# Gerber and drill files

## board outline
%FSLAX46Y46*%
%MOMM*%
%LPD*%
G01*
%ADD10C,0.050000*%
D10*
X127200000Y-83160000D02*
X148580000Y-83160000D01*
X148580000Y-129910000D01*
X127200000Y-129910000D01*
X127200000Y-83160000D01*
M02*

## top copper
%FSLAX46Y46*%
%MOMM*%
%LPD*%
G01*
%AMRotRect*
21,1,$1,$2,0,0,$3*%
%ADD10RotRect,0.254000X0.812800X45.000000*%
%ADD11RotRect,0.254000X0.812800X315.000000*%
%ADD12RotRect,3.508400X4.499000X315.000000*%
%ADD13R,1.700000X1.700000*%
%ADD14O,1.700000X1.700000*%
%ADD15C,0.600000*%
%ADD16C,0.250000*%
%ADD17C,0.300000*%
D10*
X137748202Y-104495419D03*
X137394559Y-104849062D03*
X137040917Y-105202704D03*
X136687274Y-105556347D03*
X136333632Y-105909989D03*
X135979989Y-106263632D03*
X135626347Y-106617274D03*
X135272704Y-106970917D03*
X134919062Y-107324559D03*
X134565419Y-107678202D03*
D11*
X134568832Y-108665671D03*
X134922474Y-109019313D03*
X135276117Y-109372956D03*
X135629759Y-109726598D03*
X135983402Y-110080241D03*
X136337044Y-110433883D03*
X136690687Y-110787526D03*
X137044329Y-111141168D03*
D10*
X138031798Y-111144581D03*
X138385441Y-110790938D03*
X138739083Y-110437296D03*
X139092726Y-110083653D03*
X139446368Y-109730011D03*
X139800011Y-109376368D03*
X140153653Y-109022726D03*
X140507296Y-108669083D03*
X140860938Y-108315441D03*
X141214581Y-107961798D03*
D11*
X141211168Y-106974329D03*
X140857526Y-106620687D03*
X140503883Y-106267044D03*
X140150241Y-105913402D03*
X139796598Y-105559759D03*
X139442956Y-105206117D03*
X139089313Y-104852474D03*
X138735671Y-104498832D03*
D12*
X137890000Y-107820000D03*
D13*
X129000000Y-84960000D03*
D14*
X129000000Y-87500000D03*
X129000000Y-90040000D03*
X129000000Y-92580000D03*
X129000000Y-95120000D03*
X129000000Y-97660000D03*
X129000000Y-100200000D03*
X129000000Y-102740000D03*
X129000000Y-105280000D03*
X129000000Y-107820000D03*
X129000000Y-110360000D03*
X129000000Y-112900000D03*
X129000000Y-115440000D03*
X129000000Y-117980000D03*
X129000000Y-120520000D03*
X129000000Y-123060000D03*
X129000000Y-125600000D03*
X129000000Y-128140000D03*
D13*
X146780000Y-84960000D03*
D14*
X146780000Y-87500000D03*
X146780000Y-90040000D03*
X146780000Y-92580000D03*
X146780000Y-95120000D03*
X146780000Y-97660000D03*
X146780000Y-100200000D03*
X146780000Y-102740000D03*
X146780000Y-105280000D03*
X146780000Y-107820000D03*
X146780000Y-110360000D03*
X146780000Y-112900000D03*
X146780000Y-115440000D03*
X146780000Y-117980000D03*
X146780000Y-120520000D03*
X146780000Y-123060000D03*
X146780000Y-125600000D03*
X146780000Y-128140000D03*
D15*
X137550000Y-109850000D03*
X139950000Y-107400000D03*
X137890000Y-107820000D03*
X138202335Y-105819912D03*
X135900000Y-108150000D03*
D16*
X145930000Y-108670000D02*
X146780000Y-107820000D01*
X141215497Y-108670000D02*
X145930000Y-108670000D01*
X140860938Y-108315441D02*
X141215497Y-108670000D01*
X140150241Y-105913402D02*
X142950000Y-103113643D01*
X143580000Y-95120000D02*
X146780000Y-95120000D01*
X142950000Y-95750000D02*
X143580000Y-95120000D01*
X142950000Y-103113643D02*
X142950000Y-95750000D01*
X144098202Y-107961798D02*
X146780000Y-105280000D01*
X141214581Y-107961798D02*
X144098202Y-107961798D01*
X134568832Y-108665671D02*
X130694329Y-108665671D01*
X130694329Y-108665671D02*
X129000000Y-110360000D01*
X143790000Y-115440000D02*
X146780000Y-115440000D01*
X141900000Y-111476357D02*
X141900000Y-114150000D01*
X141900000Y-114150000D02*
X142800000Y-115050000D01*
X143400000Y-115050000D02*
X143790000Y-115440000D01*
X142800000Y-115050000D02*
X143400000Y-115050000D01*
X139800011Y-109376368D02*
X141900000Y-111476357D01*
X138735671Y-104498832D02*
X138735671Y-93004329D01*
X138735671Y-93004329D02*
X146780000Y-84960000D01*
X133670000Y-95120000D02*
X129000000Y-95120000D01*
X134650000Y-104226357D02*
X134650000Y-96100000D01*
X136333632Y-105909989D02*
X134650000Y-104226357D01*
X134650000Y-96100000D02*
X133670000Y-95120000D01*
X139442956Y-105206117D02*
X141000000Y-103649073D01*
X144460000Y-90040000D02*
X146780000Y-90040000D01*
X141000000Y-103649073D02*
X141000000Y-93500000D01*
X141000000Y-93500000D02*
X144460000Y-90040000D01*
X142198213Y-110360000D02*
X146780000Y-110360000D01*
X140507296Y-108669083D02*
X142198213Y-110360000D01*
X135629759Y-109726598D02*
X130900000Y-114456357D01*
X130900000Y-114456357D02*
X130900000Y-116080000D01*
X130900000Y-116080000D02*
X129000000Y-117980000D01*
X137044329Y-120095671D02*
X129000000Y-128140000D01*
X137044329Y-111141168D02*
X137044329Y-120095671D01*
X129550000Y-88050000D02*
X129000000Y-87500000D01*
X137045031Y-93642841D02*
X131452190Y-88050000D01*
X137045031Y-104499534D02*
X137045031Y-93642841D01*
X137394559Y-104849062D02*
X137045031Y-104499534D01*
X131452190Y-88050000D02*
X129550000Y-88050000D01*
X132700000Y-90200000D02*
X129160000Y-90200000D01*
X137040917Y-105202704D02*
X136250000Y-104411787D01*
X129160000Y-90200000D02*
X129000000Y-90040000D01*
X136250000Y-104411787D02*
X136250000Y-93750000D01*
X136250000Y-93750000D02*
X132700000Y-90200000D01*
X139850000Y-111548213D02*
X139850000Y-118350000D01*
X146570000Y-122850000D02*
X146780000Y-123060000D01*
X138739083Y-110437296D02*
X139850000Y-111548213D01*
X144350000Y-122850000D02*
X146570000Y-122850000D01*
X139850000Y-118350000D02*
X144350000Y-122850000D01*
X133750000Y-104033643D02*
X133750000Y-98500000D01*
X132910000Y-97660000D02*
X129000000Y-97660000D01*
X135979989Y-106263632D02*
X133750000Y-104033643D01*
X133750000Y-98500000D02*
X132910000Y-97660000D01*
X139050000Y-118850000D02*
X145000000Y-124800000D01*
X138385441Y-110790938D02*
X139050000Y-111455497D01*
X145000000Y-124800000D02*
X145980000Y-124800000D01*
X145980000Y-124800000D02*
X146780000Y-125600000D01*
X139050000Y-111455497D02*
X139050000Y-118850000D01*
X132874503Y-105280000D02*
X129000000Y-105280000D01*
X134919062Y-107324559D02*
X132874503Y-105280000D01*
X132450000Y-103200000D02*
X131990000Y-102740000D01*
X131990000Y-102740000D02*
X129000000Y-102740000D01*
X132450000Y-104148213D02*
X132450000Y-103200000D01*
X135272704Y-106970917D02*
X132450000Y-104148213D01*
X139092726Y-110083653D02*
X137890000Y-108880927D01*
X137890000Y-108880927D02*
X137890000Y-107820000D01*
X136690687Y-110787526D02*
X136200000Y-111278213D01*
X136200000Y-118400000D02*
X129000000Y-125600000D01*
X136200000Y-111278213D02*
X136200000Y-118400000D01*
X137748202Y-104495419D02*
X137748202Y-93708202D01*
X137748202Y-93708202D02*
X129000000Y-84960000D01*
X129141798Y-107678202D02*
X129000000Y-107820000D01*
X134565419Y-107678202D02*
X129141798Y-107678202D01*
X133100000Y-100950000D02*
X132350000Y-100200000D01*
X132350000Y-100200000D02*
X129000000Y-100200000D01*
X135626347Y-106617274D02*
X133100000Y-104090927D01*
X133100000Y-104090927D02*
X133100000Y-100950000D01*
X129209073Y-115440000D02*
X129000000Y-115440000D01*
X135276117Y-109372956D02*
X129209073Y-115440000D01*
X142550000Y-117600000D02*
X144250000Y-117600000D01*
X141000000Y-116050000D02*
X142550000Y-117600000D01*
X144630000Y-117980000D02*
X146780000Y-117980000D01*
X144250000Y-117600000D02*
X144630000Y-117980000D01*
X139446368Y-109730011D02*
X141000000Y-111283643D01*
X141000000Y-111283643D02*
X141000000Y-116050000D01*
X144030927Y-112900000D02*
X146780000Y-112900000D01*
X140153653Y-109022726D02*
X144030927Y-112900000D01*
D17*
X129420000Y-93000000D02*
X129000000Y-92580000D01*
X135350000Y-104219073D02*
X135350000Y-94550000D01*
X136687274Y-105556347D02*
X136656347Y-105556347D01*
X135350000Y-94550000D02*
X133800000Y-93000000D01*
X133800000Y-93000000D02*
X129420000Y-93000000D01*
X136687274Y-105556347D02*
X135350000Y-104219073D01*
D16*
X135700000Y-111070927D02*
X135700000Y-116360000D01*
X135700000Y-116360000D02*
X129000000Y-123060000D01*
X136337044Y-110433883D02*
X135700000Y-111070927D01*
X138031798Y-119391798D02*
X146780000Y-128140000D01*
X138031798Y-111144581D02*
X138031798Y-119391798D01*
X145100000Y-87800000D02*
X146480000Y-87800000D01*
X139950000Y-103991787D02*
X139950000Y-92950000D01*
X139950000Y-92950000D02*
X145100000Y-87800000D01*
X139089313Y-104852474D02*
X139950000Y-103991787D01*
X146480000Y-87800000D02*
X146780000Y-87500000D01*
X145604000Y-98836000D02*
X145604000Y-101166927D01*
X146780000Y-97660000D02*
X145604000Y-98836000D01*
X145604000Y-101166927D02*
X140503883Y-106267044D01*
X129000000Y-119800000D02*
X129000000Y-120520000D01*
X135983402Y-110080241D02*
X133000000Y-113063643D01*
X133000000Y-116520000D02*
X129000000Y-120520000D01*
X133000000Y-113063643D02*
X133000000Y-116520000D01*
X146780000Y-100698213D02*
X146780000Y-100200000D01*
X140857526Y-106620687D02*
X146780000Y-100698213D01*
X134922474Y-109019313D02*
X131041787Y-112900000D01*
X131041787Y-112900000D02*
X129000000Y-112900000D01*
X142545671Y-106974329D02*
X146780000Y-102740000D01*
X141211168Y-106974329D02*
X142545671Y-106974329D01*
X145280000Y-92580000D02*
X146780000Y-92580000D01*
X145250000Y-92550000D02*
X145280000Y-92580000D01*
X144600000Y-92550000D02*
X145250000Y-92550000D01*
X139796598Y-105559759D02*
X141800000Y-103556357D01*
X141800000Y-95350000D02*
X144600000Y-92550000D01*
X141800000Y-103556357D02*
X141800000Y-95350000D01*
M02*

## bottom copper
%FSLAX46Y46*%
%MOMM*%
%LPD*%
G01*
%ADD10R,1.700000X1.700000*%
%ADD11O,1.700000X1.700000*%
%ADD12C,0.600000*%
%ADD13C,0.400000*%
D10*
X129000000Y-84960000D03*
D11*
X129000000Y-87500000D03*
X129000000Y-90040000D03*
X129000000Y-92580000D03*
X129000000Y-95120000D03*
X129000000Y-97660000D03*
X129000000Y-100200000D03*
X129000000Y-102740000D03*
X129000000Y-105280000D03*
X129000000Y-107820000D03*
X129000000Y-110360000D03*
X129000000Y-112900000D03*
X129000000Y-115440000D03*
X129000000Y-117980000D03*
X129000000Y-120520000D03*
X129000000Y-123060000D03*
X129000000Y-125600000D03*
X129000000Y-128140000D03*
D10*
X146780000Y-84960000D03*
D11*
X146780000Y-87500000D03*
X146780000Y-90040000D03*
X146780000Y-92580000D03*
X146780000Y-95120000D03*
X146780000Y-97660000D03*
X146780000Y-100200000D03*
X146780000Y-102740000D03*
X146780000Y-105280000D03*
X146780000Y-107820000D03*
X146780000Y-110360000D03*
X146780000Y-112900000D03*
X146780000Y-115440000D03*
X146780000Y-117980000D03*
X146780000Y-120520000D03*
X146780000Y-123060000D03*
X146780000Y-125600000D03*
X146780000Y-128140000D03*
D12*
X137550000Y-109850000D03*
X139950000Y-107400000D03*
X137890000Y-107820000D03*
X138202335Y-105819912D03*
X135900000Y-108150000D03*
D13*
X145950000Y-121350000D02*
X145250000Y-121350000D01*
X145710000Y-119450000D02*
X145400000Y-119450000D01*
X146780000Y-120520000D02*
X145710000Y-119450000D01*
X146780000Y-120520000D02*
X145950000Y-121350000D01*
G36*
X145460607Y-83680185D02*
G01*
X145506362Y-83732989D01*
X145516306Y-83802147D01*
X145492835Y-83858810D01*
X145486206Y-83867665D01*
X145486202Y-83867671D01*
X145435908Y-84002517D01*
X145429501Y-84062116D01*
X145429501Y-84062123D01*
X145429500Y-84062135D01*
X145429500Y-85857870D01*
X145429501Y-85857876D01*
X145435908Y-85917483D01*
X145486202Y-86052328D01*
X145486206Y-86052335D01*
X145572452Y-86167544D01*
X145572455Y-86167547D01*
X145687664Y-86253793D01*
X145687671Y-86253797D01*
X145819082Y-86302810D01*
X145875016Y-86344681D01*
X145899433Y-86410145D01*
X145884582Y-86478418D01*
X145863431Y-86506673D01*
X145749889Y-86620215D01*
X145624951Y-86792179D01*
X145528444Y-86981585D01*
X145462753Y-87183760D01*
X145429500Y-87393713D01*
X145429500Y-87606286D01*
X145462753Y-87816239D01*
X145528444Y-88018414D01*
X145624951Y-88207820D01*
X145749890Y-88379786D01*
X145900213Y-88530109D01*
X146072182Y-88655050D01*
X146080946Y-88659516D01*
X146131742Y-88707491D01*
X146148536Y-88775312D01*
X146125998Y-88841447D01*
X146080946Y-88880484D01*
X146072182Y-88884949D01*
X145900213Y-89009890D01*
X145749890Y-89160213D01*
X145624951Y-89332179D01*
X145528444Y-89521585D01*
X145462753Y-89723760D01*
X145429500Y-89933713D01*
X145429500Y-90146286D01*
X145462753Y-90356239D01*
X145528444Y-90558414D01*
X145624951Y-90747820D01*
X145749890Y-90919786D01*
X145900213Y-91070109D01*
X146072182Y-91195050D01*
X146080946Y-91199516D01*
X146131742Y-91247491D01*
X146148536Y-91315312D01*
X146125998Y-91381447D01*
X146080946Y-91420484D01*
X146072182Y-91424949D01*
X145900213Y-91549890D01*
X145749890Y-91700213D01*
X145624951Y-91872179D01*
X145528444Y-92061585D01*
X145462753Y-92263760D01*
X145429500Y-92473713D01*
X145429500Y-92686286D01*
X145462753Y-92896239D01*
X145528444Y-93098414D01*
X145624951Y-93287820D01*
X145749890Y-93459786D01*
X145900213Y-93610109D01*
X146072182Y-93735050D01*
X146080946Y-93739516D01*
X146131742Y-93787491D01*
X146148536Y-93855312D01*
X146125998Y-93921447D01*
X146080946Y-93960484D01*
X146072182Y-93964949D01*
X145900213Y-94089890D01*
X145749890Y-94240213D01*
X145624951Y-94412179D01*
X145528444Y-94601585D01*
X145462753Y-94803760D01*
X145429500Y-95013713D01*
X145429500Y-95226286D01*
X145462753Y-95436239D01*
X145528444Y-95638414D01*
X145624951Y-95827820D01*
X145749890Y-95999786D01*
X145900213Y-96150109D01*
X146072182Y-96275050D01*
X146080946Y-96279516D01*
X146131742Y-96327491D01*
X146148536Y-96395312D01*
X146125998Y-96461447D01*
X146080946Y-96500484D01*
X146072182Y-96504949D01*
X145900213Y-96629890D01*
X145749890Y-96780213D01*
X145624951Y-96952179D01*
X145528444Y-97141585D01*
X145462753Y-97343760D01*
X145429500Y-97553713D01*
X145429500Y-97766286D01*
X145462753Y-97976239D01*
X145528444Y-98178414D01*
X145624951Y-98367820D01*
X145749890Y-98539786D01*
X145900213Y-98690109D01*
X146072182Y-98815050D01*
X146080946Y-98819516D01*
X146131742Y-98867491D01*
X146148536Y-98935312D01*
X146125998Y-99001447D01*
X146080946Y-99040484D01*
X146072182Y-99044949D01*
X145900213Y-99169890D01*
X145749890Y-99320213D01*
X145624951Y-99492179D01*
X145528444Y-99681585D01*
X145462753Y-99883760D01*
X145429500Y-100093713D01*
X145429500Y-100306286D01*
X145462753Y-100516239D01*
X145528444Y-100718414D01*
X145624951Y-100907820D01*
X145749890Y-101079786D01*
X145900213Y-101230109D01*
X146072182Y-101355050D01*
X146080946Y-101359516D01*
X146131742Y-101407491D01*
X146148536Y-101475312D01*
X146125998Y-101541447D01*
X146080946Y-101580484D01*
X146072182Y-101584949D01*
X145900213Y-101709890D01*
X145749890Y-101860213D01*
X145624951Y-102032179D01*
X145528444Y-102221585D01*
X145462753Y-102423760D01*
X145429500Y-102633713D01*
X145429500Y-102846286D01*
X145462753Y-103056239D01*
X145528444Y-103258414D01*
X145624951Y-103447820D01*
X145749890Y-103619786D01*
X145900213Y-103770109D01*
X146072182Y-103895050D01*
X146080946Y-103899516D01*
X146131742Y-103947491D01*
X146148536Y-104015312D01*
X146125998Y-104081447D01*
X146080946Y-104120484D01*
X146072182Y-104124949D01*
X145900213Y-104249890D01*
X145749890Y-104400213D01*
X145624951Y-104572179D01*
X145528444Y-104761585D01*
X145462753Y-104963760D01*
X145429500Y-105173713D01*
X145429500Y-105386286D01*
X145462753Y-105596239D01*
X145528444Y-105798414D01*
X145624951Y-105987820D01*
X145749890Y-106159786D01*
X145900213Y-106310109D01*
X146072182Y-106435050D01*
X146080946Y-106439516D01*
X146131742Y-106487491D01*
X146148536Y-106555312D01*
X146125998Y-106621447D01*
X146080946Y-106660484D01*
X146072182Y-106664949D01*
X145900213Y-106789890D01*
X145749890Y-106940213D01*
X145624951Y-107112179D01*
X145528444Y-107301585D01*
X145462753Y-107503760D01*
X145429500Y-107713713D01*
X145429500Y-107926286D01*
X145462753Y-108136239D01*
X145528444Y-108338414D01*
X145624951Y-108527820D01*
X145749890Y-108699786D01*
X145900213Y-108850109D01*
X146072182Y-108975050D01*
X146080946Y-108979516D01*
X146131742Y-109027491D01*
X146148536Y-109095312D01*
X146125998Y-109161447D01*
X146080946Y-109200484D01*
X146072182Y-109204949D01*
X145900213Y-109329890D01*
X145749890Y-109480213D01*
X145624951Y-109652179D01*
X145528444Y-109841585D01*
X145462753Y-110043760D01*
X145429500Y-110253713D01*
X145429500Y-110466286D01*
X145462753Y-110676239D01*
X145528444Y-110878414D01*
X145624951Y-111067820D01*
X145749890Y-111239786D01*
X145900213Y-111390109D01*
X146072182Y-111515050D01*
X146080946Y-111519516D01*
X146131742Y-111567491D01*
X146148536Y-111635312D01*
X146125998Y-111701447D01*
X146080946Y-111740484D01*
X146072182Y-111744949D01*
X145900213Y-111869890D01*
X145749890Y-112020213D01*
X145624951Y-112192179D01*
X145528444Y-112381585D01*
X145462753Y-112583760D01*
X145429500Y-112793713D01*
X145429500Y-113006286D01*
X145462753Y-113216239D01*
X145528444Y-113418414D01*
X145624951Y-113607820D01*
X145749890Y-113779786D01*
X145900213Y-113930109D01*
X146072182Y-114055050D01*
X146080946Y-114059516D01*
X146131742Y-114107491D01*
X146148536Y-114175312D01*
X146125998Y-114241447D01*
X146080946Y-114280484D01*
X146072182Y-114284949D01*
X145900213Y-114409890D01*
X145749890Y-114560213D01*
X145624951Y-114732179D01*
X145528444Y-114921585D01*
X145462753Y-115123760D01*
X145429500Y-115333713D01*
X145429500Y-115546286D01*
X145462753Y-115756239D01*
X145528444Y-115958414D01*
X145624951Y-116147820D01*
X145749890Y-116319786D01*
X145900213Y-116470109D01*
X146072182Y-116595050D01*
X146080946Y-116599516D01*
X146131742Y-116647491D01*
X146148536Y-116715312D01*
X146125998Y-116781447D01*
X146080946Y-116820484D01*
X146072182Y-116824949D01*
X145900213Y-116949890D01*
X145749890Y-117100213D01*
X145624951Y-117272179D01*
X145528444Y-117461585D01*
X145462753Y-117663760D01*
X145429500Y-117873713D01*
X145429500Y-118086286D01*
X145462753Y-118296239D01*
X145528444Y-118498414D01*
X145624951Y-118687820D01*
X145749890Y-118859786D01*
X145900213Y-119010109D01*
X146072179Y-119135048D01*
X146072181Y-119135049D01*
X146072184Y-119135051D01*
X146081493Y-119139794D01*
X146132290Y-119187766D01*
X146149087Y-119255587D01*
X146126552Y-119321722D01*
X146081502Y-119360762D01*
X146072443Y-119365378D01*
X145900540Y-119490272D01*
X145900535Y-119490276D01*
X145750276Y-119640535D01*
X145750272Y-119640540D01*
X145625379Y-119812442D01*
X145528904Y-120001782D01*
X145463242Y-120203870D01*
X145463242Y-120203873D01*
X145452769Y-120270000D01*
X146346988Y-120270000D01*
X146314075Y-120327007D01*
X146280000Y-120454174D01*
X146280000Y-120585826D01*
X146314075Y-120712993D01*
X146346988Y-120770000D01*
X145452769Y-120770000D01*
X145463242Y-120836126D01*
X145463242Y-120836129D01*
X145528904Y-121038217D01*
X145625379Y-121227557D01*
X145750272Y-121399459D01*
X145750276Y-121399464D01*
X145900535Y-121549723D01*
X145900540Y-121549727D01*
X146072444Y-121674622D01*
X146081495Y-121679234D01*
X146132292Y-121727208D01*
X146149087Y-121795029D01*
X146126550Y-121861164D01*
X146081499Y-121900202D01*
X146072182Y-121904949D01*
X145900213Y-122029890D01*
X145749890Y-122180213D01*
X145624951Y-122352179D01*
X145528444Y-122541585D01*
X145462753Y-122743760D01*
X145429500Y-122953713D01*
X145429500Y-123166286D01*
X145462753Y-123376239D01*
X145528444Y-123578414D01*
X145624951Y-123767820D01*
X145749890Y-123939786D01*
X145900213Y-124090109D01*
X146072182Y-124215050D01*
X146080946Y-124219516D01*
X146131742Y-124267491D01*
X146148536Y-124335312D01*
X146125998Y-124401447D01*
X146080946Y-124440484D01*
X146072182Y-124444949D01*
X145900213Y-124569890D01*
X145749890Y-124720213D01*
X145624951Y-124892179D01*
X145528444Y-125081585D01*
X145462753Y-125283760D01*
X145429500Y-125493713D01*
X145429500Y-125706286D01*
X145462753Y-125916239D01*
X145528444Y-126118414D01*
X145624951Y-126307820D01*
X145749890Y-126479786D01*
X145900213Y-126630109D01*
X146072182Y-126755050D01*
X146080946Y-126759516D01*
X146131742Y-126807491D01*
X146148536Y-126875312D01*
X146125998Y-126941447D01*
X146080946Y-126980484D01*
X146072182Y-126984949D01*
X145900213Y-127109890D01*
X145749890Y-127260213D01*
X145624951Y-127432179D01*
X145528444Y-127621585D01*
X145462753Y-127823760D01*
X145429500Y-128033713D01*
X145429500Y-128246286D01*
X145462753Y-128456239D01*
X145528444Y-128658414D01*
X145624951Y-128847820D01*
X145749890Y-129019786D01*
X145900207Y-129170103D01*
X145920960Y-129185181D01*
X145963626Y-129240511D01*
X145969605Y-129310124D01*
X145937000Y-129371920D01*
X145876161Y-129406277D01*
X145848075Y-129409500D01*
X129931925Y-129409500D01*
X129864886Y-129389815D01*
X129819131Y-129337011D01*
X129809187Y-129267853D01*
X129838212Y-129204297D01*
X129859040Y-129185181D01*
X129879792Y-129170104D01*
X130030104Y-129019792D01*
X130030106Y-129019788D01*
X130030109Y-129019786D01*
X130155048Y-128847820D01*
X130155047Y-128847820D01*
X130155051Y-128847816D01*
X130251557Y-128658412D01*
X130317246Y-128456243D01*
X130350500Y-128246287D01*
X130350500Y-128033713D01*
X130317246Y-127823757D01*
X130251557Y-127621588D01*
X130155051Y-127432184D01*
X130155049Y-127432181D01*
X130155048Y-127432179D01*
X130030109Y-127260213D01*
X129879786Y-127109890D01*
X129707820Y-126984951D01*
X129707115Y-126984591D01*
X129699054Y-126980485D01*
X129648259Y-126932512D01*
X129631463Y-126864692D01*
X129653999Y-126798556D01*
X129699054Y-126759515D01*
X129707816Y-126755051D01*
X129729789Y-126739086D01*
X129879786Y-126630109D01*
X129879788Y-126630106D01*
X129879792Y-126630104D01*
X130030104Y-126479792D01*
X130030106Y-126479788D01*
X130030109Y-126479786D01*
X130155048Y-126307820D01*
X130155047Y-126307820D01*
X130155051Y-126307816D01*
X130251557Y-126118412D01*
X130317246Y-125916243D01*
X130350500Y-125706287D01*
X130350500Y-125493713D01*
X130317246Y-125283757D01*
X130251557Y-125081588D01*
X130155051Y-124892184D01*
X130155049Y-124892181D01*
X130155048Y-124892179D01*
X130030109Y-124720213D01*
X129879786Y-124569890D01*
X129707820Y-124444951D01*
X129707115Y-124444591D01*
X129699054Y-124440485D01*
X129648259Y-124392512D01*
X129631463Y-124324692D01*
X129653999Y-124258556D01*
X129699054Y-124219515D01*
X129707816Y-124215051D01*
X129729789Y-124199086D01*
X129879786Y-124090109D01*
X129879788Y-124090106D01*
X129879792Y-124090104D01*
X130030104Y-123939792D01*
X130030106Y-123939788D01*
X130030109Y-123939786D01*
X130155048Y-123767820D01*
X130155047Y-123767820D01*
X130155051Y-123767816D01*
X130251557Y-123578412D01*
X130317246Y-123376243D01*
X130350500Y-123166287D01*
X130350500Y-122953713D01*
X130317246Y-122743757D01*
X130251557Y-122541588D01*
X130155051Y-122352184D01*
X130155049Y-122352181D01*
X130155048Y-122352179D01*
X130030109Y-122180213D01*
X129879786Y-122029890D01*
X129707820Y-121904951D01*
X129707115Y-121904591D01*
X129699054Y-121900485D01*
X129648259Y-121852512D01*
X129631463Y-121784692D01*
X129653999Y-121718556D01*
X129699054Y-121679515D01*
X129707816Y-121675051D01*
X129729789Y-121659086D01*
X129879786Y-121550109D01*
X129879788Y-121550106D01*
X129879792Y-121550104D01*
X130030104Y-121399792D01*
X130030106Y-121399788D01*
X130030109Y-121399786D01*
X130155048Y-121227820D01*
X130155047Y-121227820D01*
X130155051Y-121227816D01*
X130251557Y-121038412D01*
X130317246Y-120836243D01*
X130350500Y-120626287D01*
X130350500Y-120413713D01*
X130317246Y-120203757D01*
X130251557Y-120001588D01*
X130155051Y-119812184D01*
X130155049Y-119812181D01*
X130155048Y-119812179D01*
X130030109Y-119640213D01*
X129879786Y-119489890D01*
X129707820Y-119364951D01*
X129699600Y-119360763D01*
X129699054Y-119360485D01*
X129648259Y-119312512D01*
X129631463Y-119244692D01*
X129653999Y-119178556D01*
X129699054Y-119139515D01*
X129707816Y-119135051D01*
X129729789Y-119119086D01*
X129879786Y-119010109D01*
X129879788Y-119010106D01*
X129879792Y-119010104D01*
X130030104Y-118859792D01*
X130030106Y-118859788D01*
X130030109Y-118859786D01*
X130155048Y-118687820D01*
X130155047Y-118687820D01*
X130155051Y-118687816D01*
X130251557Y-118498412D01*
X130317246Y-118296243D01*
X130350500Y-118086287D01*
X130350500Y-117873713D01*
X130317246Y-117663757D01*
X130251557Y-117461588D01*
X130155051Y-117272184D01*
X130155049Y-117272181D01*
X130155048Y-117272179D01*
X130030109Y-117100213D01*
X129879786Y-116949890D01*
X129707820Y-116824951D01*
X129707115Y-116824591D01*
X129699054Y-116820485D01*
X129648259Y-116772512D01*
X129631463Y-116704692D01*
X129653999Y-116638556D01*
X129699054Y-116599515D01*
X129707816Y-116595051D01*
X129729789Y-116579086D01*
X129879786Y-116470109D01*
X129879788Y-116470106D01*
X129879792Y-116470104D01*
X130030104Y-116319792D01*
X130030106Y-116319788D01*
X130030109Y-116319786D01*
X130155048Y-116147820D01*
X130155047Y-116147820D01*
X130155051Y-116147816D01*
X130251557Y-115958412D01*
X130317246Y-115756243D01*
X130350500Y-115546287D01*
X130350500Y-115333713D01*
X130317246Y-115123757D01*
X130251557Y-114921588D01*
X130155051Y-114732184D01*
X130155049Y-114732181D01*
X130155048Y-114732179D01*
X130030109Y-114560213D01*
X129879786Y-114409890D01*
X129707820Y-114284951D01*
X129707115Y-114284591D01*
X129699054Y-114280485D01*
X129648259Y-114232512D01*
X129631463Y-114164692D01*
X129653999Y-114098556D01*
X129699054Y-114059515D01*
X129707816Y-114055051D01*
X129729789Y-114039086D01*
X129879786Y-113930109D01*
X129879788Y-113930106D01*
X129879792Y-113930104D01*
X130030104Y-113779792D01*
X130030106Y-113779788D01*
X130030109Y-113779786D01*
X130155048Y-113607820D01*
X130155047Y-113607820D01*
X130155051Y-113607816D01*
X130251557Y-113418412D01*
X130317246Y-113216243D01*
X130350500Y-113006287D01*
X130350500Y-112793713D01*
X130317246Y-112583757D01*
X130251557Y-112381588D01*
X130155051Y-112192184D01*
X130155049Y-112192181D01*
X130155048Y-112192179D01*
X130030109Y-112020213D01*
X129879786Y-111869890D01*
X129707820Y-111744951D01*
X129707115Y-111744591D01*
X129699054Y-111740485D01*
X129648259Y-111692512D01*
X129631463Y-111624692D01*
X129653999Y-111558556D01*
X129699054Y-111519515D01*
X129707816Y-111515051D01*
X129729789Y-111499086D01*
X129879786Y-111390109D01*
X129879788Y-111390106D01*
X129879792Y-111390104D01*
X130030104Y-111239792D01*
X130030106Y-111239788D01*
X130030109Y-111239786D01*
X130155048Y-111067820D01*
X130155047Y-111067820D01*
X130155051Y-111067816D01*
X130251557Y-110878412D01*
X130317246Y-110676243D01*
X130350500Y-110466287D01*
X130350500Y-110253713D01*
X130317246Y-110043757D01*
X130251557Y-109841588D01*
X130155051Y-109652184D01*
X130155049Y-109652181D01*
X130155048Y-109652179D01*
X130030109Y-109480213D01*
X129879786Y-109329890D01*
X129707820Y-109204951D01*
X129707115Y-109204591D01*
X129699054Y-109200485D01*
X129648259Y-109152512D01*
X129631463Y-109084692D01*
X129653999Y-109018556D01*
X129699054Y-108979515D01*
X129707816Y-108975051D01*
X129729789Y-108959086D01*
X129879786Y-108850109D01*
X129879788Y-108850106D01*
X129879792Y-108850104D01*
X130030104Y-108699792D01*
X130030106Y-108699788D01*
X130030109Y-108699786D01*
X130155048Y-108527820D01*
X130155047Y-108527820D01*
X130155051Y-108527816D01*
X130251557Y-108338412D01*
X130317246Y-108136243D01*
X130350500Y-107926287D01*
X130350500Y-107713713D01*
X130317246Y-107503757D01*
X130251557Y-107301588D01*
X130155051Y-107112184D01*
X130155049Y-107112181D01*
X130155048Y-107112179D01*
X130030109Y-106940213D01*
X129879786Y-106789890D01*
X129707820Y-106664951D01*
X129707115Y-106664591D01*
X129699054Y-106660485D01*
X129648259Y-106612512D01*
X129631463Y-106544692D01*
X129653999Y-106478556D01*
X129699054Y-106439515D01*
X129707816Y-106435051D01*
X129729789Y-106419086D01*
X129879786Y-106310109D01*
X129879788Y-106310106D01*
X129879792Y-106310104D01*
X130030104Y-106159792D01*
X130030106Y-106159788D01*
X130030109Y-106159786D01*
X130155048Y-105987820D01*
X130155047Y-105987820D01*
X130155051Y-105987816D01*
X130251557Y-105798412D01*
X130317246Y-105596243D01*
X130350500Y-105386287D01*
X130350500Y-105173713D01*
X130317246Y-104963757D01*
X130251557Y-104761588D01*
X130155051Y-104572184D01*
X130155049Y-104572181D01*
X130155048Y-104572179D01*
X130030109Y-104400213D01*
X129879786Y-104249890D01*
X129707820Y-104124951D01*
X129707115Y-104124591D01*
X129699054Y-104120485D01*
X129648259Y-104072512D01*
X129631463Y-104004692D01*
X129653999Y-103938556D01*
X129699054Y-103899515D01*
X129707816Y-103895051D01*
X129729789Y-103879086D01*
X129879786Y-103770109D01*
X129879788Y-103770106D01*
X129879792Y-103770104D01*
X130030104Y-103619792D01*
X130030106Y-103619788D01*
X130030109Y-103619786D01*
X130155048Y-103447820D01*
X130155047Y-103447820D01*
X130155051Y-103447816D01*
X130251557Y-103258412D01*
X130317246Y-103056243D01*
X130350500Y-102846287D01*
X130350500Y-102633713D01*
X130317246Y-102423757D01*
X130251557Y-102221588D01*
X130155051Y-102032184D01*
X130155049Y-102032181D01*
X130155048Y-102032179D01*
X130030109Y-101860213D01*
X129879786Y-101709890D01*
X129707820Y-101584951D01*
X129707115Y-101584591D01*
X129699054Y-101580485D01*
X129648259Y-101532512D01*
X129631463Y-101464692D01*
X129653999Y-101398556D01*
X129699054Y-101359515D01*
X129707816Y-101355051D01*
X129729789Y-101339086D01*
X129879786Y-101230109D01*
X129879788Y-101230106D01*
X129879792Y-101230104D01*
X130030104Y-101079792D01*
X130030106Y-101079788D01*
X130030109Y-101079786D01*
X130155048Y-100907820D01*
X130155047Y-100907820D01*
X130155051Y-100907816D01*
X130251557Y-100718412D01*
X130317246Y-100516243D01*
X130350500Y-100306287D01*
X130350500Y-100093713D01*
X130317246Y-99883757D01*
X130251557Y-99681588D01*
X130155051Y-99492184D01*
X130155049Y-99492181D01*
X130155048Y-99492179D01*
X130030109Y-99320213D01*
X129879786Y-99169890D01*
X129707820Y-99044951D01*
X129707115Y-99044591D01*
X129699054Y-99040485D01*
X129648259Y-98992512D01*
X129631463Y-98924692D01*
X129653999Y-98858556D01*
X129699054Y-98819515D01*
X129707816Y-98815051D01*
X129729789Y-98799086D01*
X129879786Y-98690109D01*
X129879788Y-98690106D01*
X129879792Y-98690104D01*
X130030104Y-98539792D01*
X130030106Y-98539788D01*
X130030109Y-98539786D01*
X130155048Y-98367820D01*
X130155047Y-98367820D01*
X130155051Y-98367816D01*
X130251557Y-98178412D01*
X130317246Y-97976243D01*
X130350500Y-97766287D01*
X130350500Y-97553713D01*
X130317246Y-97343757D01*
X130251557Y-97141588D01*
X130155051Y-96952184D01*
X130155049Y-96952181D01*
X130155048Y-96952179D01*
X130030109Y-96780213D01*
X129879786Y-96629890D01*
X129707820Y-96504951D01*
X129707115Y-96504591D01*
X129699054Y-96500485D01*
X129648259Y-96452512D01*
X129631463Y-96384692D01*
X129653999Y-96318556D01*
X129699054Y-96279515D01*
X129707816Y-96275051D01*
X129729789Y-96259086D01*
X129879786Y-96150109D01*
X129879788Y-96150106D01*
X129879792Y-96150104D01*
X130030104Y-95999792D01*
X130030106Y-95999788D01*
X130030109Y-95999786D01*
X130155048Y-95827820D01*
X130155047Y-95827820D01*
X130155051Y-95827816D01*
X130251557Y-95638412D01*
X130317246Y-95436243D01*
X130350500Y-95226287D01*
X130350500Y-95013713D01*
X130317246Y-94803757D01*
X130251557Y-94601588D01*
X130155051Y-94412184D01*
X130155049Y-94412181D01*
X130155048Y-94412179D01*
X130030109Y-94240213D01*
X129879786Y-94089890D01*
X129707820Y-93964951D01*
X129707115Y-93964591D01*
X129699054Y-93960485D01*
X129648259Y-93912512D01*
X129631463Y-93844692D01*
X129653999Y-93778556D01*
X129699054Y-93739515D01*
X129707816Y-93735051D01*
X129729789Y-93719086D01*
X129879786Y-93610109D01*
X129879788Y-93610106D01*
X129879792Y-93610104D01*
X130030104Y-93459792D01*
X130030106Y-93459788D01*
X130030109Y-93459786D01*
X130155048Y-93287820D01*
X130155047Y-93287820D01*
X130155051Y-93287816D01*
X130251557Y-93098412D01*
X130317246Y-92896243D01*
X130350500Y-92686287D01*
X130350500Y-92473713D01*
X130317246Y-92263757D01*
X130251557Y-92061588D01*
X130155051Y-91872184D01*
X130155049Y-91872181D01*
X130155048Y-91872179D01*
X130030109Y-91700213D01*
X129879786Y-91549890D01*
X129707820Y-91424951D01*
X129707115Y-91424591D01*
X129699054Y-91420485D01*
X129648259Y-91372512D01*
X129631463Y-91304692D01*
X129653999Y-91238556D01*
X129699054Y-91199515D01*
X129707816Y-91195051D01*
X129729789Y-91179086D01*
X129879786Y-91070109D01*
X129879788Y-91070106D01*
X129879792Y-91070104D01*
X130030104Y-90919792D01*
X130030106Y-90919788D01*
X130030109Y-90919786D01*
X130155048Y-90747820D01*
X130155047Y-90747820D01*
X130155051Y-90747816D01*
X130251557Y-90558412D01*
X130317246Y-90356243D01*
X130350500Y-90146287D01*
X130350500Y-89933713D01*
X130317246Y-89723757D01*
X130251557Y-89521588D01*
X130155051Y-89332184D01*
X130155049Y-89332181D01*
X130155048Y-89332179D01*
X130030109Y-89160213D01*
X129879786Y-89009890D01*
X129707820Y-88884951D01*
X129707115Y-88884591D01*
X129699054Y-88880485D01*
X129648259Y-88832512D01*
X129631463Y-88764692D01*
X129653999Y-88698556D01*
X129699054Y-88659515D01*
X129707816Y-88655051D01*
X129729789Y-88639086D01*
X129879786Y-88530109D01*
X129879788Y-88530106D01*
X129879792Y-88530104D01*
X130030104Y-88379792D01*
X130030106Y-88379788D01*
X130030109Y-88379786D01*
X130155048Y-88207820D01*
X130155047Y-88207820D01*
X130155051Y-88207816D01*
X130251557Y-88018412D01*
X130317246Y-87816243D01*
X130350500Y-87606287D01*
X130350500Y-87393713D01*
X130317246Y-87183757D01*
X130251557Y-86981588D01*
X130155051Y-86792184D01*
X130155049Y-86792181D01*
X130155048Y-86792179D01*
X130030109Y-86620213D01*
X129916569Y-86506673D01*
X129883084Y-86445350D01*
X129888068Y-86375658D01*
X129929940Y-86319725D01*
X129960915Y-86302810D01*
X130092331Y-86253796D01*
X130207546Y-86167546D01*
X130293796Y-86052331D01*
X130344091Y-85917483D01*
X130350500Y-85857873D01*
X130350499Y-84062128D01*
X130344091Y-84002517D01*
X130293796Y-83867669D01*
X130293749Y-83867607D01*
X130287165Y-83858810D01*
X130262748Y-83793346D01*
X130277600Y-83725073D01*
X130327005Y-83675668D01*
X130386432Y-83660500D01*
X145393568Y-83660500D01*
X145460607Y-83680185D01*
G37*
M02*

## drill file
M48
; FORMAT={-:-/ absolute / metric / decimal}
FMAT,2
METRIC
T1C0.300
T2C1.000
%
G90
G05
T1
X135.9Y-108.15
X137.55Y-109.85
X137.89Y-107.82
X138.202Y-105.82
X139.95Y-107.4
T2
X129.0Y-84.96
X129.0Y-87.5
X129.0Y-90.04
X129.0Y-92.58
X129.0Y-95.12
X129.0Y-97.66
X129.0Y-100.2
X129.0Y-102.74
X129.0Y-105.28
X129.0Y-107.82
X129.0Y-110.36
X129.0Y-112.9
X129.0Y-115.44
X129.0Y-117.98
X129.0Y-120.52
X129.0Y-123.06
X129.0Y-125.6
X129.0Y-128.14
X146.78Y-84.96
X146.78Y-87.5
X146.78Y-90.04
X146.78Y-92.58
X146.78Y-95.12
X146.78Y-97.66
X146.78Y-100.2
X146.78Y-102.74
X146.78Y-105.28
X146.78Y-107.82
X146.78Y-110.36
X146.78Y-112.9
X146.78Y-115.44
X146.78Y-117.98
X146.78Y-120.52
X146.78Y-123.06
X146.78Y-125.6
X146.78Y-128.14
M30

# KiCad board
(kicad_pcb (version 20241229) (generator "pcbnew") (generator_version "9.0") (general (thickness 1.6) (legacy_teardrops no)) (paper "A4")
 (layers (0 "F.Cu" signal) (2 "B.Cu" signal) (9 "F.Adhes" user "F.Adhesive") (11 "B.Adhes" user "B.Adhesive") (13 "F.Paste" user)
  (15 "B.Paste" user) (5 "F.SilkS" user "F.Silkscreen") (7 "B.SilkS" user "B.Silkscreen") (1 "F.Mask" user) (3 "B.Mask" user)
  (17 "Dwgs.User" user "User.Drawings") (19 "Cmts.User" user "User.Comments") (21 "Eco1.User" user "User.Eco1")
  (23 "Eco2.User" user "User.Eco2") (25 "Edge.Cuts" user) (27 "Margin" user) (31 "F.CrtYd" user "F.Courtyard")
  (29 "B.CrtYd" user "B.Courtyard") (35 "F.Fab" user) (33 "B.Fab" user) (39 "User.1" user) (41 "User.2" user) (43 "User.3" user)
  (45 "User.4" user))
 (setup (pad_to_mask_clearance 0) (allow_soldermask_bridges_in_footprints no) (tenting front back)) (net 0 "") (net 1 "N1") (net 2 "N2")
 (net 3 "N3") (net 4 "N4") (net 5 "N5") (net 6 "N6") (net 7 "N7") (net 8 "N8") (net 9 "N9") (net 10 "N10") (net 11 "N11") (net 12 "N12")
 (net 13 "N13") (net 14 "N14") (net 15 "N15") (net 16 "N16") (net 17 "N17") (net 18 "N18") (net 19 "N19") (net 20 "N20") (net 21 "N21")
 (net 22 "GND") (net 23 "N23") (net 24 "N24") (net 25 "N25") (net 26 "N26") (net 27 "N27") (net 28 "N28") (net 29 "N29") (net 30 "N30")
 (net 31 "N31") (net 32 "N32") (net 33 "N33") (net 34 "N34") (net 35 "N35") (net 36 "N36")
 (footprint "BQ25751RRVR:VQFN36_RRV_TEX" (layer "F.Cu") (at 137.89 107.82 -45)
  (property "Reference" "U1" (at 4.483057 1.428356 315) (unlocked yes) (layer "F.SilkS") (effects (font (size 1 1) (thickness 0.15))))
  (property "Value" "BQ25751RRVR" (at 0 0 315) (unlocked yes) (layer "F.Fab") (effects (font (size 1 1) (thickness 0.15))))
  (pad "1" smd rect (at -2.4511 -2.250567 45) (size 0.254 0.8128) (layers "F.Cu" "F.Mask" "F.Paste") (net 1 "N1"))
  (pad "2" smd rect (at -2.4511 -1.750441 45) (size 0.254 0.8128) (layers "F.Cu" "F.Mask" "F.Paste") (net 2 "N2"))
  (pad "3" smd rect (at -2.4511 -1.250315 45) (size 0.254 0.8128) (layers "F.Cu" "F.Mask" "F.Paste") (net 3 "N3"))
  (pad "4" smd rect (at -2.4511 -0.750189 45) (size 0.254 0.8128) (layers "F.Cu" "F.Mask" "F.Paste") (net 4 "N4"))
  (pad "5" smd rect (at -2.4511 -0.250063 45) (size 0.254 0.8128) (layers "F.Cu" "F.Mask" "F.Paste") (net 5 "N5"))
  (pad "6" smd rect (at -2.4511 0.250063 45) (size 0.254 0.8128) (layers "F.Cu" "F.Mask" "F.Paste") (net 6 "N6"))
  (pad "7" smd rect (at -2.4511 0.750189 45) (size 0.254 0.8128) (layers "F.Cu" "F.Mask" "F.Paste") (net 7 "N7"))
  (pad "8" smd rect (at -2.4511 1.250315 45) (size 0.254 0.8128) (layers "F.Cu" "F.Mask" "F.Paste") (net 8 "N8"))
  (pad "9" smd rect (at -2.4511 1.750441 45) (size 0.254 0.8128) (layers "F.Cu" "F.Mask" "F.Paste") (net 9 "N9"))
  (pad "10" smd rect (at -2.4511 2.250567 45) (size 0.254 0.8128) (layers "F.Cu" "F.Mask" "F.Paste") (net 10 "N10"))
  (pad "11" smd rect (at -1.750441 2.9464 315) (size 0.254 0.8128) (layers "F.Cu" "F.Mask" "F.Paste") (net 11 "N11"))
  (pad "12" smd rect (at -1.250315 2.9464 315) (size 0.254 0.8128) (layers "F.Cu" "F.Mask" "F.Paste") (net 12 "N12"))
  (pad "13" smd rect (at -0.750189 2.9464 315) (size 0.254 0.8128) (layers "F.Cu" "F.Mask" "F.Paste") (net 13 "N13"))
  (pad "14" smd rect (at -0.250063 2.9464 315) (size 0.254 0.8128) (layers "F.Cu" "F.Mask" "F.Paste") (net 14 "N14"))
  (pad "15" smd rect (at 0.250063 2.9464 315) (size 0.254 0.8128) (layers "F.Cu" "F.Mask" "F.Paste") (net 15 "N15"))
  (pad "16" smd rect (at 0.750189 2.9464 315) (size 0.254 0.8128) (layers "F.Cu" "F.Mask" "F.Paste") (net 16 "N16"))
  (pad "17" smd rect (at 1.250315 2.9464 315) (size 0.254 0.8128) (layers "F.Cu" "F.Mask" "F.Paste") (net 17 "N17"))
  (pad "18" smd rect (at 1.750441 2.9464 315) (size 0.254 0.8128) (layers "F.Cu" "F.Mask" "F.Paste") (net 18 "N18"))
  (pad "19" smd rect (at 2.4511 2.250567 45) (size 0.254 0.8128) (layers "F.Cu" "F.Mask" "F.Paste") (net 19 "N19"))
  (pad "20" smd rect (at 2.4511 1.750441 45) (size 0.254 0.8128) (layers "F.Cu" "F.Mask" "F.Paste") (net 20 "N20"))
  (pad "21" smd rect (at 2.4511 1.250315 45) (size 0.254 0.8128) (layers "F.Cu" "F.Mask" "F.Paste") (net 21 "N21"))
  (pad "22" smd rect (at 2.4511 0.750189 45) (size 0.254 0.8128) (layers "F.Cu" "F.Mask" "F.Paste") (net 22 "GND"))
  (pad "23" smd rect (at 2.4511 0.250063 45) (size 0.254 0.8128) (layers "F.Cu" "F.Mask" "F.Paste") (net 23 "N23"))
  (pad "24" smd rect (at 2.4511 -0.250063 45) (size 0.254 0.8128) (layers "F.Cu" "F.Mask" "F.Paste") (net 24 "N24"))
  (pad "25" smd rect (at 2.4511 -0.750189 45) (size 0.254 0.8128) (layers "F.Cu" "F.Mask" "F.Paste") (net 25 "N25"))
  (pad "26" smd rect (at 2.4511 -1.250315 45) (size 0.254 0.8128) (layers "F.Cu" "F.Mask" "F.Paste") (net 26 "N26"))
  (pad "27" smd rect (at 2.4511 -1.750441 45) (size 0.254 0.8128) (layers "F.Cu" "F.Mask" "F.Paste") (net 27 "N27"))
  (pad "28" smd rect (at 2.4511 -2.250567 45) (size 0.254 0.8128) (layers "F.Cu" "F.Mask" "F.Paste") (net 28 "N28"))
  (pad "29" smd rect (at 1.750441 -2.9464 315) (size 0.254 0.8128) (layers "F.Cu" "F.Mask" "F.Paste") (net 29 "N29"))
  (pad "30" smd rect (at 1.250315 -2.9464 315) (size 0.254 0.8128) (layers "F.Cu" "F.Mask" "F.Paste") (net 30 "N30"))
  (pad "31" smd rect (at 0.750189 -2.9464 315) (size 0.254 0.8128) (layers "F.Cu" "F.Mask" "F.Paste") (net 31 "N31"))
  (pad "32" smd rect (at 0.250063 -2.9464 315) (size 0.254 0.8128) (layers "F.Cu" "F.Mask" "F.Paste") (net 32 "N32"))
  (pad "33" smd rect (at -0.250063 -2.9464 315) (size 0.254 0.8128) (layers "F.Cu" "F.Mask" "F.Paste") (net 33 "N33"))
  (pad "34" smd rect (at -0.750189 -2.9464 315) (size 0.254 0.8128) (layers "F.Cu" "F.Mask" "F.Paste") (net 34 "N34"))
  (pad "35" smd rect (at -1.250315 -2.9464 315) (size 0.254 0.8128) (layers "F.Cu" "F.Mask" "F.Paste") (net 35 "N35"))
  (pad "36" smd rect (at -1.750441 -2.9464 315) (size 0.254 0.8128) (layers "F.Cu" "F.Mask" "F.Paste") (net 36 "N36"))
  (pad "37" smd rect (at 0 0 315) (size 3.5084 4.499) (layers "F.Cu" "F.Mask" "F.Paste") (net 22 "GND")))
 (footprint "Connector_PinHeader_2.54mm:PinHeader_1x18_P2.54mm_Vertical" (layer "F.Cu") (at 129 84.96)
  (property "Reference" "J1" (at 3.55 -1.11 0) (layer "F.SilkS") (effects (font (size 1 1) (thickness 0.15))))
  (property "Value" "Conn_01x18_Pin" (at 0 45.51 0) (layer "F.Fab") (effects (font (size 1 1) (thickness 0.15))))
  (pad "1" thru_hole rect (at 0 0) (size 1.7 1.7) (drill 1) (layers "*.Cu" "*.Mask") (remove_unused_layers no) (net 1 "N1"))
  (pad "2" thru_hole oval (at 0 2.54) (size 1.7 1.7) (drill 1) (layers "*.Cu" "*.Mask") (remove_unused_layers no) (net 2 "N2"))
  (pad "3" thru_hole oval (at 0 5.08) (size 1.7 1.7) (drill 1) (layers "*.Cu" "*.Mask") (remove_unused_layers no) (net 3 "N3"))
  (pad "4" thru_hole oval (at 0 7.62) (size 1.7 1.7) (drill 1) (layers "*.Cu" "*.Mask") (remove_unused_layers no) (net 4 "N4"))
  (pad "5" thru_hole oval (at 0 10.16) (size 1.7 1.7) (drill 1) (layers "*.Cu" "*.Mask") (remove_unused_layers no) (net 5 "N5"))
  (pad "6" thru_hole oval (at 0 12.7) (size 1.7 1.7) (drill 1) (layers "*.Cu" "*.Mask") (remove_unused_layers no) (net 6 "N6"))
  (pad "7" thru_hole oval (at 0 15.24) (size 1.7 1.7) (drill 1) (layers "*.Cu" "*.Mask") (remove_unused_layers no) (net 7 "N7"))
  (pad "8" thru_hole oval (at 0 17.78) (size 1.7 1.7) (drill 1) (layers "*.Cu" "*.Mask") (remove_unused_layers no) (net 8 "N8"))
  (pad "9" thru_hole oval (at 0 20.32) (size 1.7 1.7) (drill 1) (layers "*.Cu" "*.Mask") (remove_unused_layers no) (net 9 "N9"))
  (pad "10" thru_hole oval (at 0 22.86) (size 1.7 1.7) (drill 1) (layers "*.Cu" "*.Mask") (remove_unused_layers no) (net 10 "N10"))
  (pad "11" thru_hole oval (at 0 25.4) (size 1.7 1.7) (drill 1) (layers "*.Cu" "*.Mask") (remove_unused_layers no) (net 11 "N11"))
  (pad "12" thru_hole oval (at 0 27.94) (size 1.7 1.7) (drill 1) (layers "*.Cu" "*.Mask") (remove_unused_layers no) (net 12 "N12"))
  (pad "13" thru_hole oval (at 0 30.48) (size 1.7 1.7) (drill 1) (layers "*.Cu" "*.Mask") (remove_unused_layers no) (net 13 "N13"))
  (pad "14" thru_hole oval (at 0 33.02) (size 1.7 1.7) (drill 1) (layers "*.Cu" "*.Mask") (remove_unused_layers no) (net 14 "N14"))
  (pad "15" thru_hole oval (at 0 35.56) (size 1.7 1.7) (drill 1) (layers "*.Cu" "*.Mask") (remove_unused_layers no) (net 15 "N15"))
  (pad "16" thru_hole oval (at 0 38.1) (size 1.7 1.7) (drill 1) (layers "*.Cu" "*.Mask") (remove_unused_layers no) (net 16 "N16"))
  (pad "17" thru_hole oval (at 0 40.64) (size 1.7 1.7) (drill 1) (layers "*.Cu" "*.Mask") (remove_unused_layers no) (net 17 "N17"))
  (pad "18" thru_hole oval (at 0 43.18) (size 1.7 1.7) (drill 1) (layers "*.Cu" "*.Mask") (remove_unused_layers no) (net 18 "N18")))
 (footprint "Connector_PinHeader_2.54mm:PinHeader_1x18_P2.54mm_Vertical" (layer "F.Cu") (at 146.78 84.96)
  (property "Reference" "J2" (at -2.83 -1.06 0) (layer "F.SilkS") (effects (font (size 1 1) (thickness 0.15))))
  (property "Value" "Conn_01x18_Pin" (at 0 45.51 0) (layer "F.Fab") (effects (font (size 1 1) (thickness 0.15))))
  (pad "1" thru_hole rect (at 0 0) (size 1.7 1.7) (drill 1) (layers "*.Cu" "*.Mask") (remove_unused_layers no) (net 36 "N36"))
  (pad "2" thru_hole oval (at 0 2.54) (size 1.7 1.7) (drill 1) (layers "*.Cu" "*.Mask") (remove_unused_layers no) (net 35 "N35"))
  (pad "3" thru_hole oval (at 0 5.08) (size 1.7 1.7) (drill 1) (layers "*.Cu" "*.Mask") (remove_unused_layers no) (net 34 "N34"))
  (pad "4" thru_hole oval (at 0 7.62) (size 1.7 1.7) (drill 1) (layers "*.Cu" "*.Mask") (remove_unused_layers no) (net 33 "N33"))
  (pad "5" thru_hole oval (at 0 10.16) (size 1.7 1.7) (drill 1) (layers "*.Cu" "*.Mask") (remove_unused_layers no) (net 32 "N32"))
  (pad "6" thru_hole oval (at 0 12.7) (size 1.7 1.7) (drill 1) (layers "*.Cu" "*.Mask") (remove_unused_layers no) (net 31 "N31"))
  (pad "7" thru_hole oval (at 0 15.24) (size 1.7 1.7) (drill 1) (layers "*.Cu" "*.Mask") (remove_unused_layers no) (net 30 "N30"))
  (pad "8" thru_hole oval (at 0 17.78) (size 1.7 1.7) (drill 1) (layers "*.Cu" "*.Mask") (remove_unused_layers no) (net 29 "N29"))
  (pad "9" thru_hole oval (at 0 20.32) (size 1.7 1.7) (drill 1) (layers "*.Cu" "*.Mask") (remove_unused_layers no) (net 28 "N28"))
  (pad "10" thru_hole oval (at 0 22.86) (size 1.7 1.7) (drill 1) (layers "*.Cu" "*.Mask") (remove_unused_layers no) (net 27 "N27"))
  (pad "11" thru_hole oval (at 0 25.4) (size 1.7 1.7) (drill 1) (layers "*.Cu" "*.Mask") (remove_unused_layers no) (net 26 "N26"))
  (pad "12" thru_hole oval (at 0 27.94) (size 1.7 1.7) (drill 1) (layers "*.Cu" "*.Mask") (remove_unused_layers no) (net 25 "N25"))
  (pad "13" thru_hole oval (at 0 30.48) (size 1.7 1.7) (drill 1) (layers "*.Cu" "*.Mask") (remove_unused_layers no) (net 24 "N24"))
  (pad "14" thru_hole oval (at 0 33.02) (size 1.7 1.7) (drill 1) (layers "*.Cu" "*.Mask") (remove_unused_layers no) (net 23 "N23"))
  (pad "15" thru_hole oval (at 0 35.56) (size 1.7 1.7) (drill 1) (layers "*.Cu" "*.Mask") (remove_unused_layers no) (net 22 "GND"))
  (pad "16" thru_hole oval (at 0 38.1) (size 1.7 1.7) (drill 1) (layers "*.Cu" "*.Mask") (remove_unused_layers no) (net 21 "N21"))
  (pad "17" thru_hole oval (at 0 40.64) (size 1.7 1.7) (drill 1) (layers "*.Cu" "*.Mask") (remove_unused_layers no) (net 20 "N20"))
  (pad "18" thru_hole oval (at 0 43.18) (size 1.7 1.7) (drill 1) (layers "*.Cu" "*.Mask") (remove_unused_layers no) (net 19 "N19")))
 (gr_rect (start 127.2 83.16) (end 148.58 129.91) (stroke (width 0.05) (type default)) (fill no) (layer "Edge.Cuts"))
 (segment (start 145.93 108.67) (end 146.78 107.82) (width 0.25) (layer "F.Cu") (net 27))
 (segment (start 141.215497 108.67) (end 145.93 108.67) (width 0.25) (layer "F.Cu") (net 27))
 (segment (start 140.860938 108.315441) (end 141.215497 108.67) (width 0.25) (layer "F.Cu") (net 27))
 (segment (start 140.150241 105.913402) (end 142.95 103.113643) (width 0.25) (layer "F.Cu") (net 32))
 (segment (start 143.58 95.12) (end 146.78 95.12) (width 0.25) (layer "F.Cu") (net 32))
 (segment (start 142.95 95.75) (end 143.58 95.12) (width 0.25) (layer "F.Cu") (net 32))
 (segment (start 142.95 103.113643) (end 142.95 95.75) (width 0.25) (layer "F.Cu") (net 32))
 (segment (start 144.098202 107.961798) (end 146.78 105.28) (width 0.25) (layer "F.Cu") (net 28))
 (segment (start 141.214581 107.961798) (end 144.098202 107.961798) (width 0.25) (layer "F.Cu") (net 28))
 (segment (start 134.568832 108.665671) (end 130.694329 108.665671) (width 0.25) (layer "F.Cu") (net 11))
 (segment (start 130.694329 108.665671) (end 129 110.36) (width 0.25) (layer "F.Cu") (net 11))
 (segment (start 143.79 115.44) (end 146.78 115.44) (width 0.25) (layer "F.Cu") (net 24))
 (segment (start 141.9 111.476357) (end 141.9 114.15) (width 0.25) (layer "F.Cu") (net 24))
 (segment (start 141.9 114.15) (end 142.8 115.05) (width 0.25) (layer "F.Cu") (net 24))
 (segment (start 143.4 115.05) (end 143.79 115.44) (width 0.25) (layer "F.Cu") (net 24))
 (segment (start 142.8 115.05) (end 143.4 115.05) (width 0.25) (layer "F.Cu") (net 24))
 (segment (start 139.800011 109.376368) (end 141.9 111.476357) (width 0.25) (layer "F.Cu") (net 24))
 (segment (start 138.735671 104.498832) (end 138.735671 93.004329) (width 0.25) (layer "F.Cu") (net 36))
 (segment (start 138.735671 93.004329) (end 146.78 84.96) (width 0.25) (layer "F.Cu") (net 36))
 (segment (start 133.67 95.12) (end 129 95.12) (width 0.25) (layer "F.Cu") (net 5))
 (segment (start 134.65 104.226357) (end 134.65 96.1) (width 0.25) (layer "F.Cu") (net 5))
 (segment (start 136.333632 105.909989) (end 134.65 104.226357) (width 0.25) (layer "F.Cu") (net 5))
 (segment (start 134.65 96.1) (end 133.67 95.12) (width 0.25) (layer "F.Cu") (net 5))
 (segment (start 139.442956 105.206117) (end 141 103.649073) (width 0.25) (layer "F.Cu") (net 34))
 (segment (start 144.46 90.04) (end 146.78 90.04) (width 0.25) (layer "F.Cu") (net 34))
 (segment (start 141 103.649073) (end 141 93.5) (width 0.25) (layer "F.Cu") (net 34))
 (segment (start 141 93.5) (end 144.46 90.04) (width 0.25) (layer "F.Cu") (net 34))
 (segment (start 142.198213 110.36) (end 146.78 110.36) (width 0.25) (layer "F.Cu") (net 26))
 (segment (start 140.507296 108.669083) (end 142.198213 110.36) (width 0.25) (layer "F.Cu") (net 26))
 (segment (start 135.629759 109.726598) (end 130.9 114.456357) (width 0.25) (layer "F.Cu") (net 14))
 (segment (start 130.9 114.456357) (end 130.9 116.08) (width 0.25) (layer "F.Cu") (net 14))
 (segment (start 130.9 116.08) (end 129 117.98) (width 0.25) (layer "F.Cu") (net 14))
 (segment (start 137.044329 120.095671) (end 129 128.14) (width 0.25) (layer "F.Cu") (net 18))
 (segment (start 137.044329 111.141168) (end 137.044329 120.095671) (width 0.25) (layer "F.Cu") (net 18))
 (segment (start 129.55 88.05) (end 129 87.5) (width 0.25) (layer "F.Cu") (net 2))
 (segment (start 137.045031 93.642841) (end 131.45219 88.05) (width 0.25) (layer "F.Cu") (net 2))
 (segment (start 137.045031 104.499534) (end 137.045031 93.642841) (width 0.25) (layer "F.Cu") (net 2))
 (segment (start 137.394559 104.849062) (end 137.045031 104.499534) (width 0.25) (layer "F.Cu") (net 2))
 (segment (start 131.45219 88.05) (end 129.55 88.05) (width 0.25) (layer "F.Cu") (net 2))
 (segment (start 132.7 90.2) (end 129.16 90.2) (width 0.25) (layer "F.Cu") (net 3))
 (segment (start 137.040917 105.202704) (end 136.25 104.411787) (width 0.25) (layer "F.Cu") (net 3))
 (segment (start 129.16 90.2) (end 129 90.04) (width 0.25) (layer "F.Cu") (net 3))
 (segment (start 136.25 104.411787) (end 136.25 93.75) (width 0.25) (layer "F.Cu") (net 3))
 (segment (start 136.25 93.75) (end 132.7 90.2) (width 0.25) (layer "F.Cu") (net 3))
 (segment (start 139.85 111.548213) (end 139.85 118.35) (width 0.25) (layer "F.Cu") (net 21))
 (segment (start 146.57 122.85) (end 146.78 123.06) (width 0.25) (layer "F.Cu") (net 21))
 (segment (start 138.739083 110.437296) (end 139.85 111.548213) (width 0.25) (layer "F.Cu") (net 21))
 (segment (start 144.35 122.85) (end 146.57 122.85) (width 0.25) (layer "F.Cu") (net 21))
 (segment (start 139.85 118.35) (end 144.35 122.85) (width 0.25) (layer "F.Cu") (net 21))
 (segment (start 133.75 104.033643) (end 133.75 98.5) (width 0.25) (layer "F.Cu") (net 6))
 (segment (start 132.91 97.66) (end 129 97.66) (width 0.25) (layer "F.Cu") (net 6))
 (segment (start 135.979989 106.263632) (end 133.75 104.033643) (width 0.25) (layer "F.Cu") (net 6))
 (segment (start 133.75 98.5) (end 132.91 97.66) (width 0.25) (layer "F.Cu") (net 6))
 (segment (start 139.05 118.85) (end 145 124.8) (width 0.25) (layer "F.Cu") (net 20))
 (segment (start 138.385441 110.790938) (end 139.05 111.455497) (width 0.25) (layer "F.Cu") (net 20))
 (segment (start 145 124.8) (end 145.98 124.8) (width 0.25) (layer "F.Cu") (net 20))
 (segment (start 145.98 124.8) (end 146.78 125.6) (width 0.25) (layer "F.Cu") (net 20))
 (segment (start 139.05 111.455497) (end 139.05 118.85) (width 0.25) (layer "F.Cu") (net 20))
 (segment (start 132.874503 105.28) (end 129 105.28) (width 0.25) (layer "F.Cu") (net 9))
 (segment (start 134.919062 107.324559) (end 132.874503 105.28) (width 0.25) (layer "F.Cu") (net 9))
 (segment (start 132.45 103.2) (end 131.99 102.74) (width 0.25) (layer "F.Cu") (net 8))
 (segment (start 131.99 102.74) (end 129 102.74) (width 0.25) (layer "F.Cu") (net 8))
 (segment (start 132.45 104.148213) (end 132.45 103.2) (width 0.25) (layer "F.Cu") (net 8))
 (segment (start 135.272704 106.970917) (end 132.45 104.148213) (width 0.25) (layer "F.Cu") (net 8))
 (segment (start 139.092726 110.083653) (end 137.89 108.880927) (width 0.25) (layer "F.Cu") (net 22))
 (segment (start 137.89 108.880927) (end 137.89 107.82) (width 0.25) (layer "F.Cu") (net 22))
 (via (at 137.55 109.85) (size 0.6) (drill 0.3) (layers "F.Cu" "B.Cu") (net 22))
 (via (at 139.95 107.4) (size 0.6) (drill 0.3) (layers "F.Cu" "B.Cu") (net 22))
 (via (at 137.89 107.82) (size 0.6) (drill 0.3) (layers "F.Cu" "B.Cu") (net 22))
 (via (at 138.202335 105.819912) (size 0.6) (drill 0.3) (layers "F.Cu" "B.Cu") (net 22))
 (via (at 135.9 108.15) (size 0.6) (drill 0.3) (layers "F.Cu" "B.Cu") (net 22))
 (segment (start 145.95 121.35) (end 145.25 121.35) (width 0.4) (layer "B.Cu") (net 22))
 (segment (start 145.71 119.45) (end 145.4 119.45) (width 0.4) (layer "B.Cu") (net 22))
 (segment (start 146.78 120.52) (end 145.71 119.45) (width 0.4) (layer "B.Cu") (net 22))
 (segment (start 146.78 120.52) (end 145.95 121.35) (width 0.4) (layer "B.Cu") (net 22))
 (segment (start 136.690687 110.787526) (end 136.2 111.278213) (width 0.25) (layer "F.Cu") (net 17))
 (segment (start 136.2 118.4) (end 129 125.6) (width 0.25) (layer "F.Cu") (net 17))
 (segment (start 136.2 111.278213) (end 136.2 118.4) (width 0.25) (layer "F.Cu") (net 17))
 (segment (start 137.748202 104.495419) (end 137.748202 93.708202) (width 0.25) (layer "F.Cu") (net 1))
 (segment (start 137.748202 93.708202) (end 129 84.96) (width 0.25) (layer "F.Cu") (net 1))
 (segment (start 129.141798 107.678202) (end 129 107.82) (width 0.25) (layer "F.Cu") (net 10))
 (segment (start 134.565419 107.678202) (end 129.141798 107.678202) (width 0.25) (layer "F.Cu") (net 10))
 (segment (start 133.1 100.95) (end 132.35 100.2) (width 0.25) (layer "F.Cu") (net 7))
 (segment (start 132.35 100.2) (end 129 100.2) (width 0.25) (layer "F.Cu") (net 7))
 (segment (start 135.626347 106.617274) (end 133.1 104.090927) (width 0.25) (layer "F.Cu") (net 7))
 (segment (start 133.1 104.090927) (end 133.1 100.95) (width 0.25) (layer "F.Cu") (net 7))
 (segment (start 129.209073 115.44) (end 129 115.44) (width 0.25) (layer "F.Cu") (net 13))
 (segment (start 135.276117 109.372956) (end 129.209073 115.44) (width 0.25) (layer "F.Cu") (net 13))
 (segment (start 142.55 117.6) (end 144.25 117.6) (width 0.25) (layer "F.Cu") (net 23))
 (segment (start 141 116.05) (end 142.55 117.6) (width 0.25) (layer "F.Cu") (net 23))
 (segment (start 144.63 117.98) (end 146.78 117.98) (width 0.25) (layer "F.Cu") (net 23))
 (segment (start 144.25 117.6) (end 144.63 117.98) (width 0.25) (layer "F.Cu") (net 23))
 (segment (start 139.446368 109.730011) (end 141 111.283643) (width 0.25) (layer "F.Cu") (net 23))
 (segment (start 141 111.283643) (end 141 116.05) (width 0.25) (layer "F.Cu") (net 23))
 (segment (start 144.030927 112.9) (end 146.78 112.9) (width 0.25) (layer "F.Cu") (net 25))
 (segment (start 140.153653 109.022726) (end 144.030927 112.9) (width 0.25) (layer "F.Cu") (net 25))
 (segment (start 129.42 93) (end 129 92.58) (width 0.3) (layer "F.Cu") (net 4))
 (segment (start 135.35 104.219073) (end 135.35 94.55) (width 0.3) (layer "F.Cu") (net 4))
 (segment (start 136.687274 105.556347) (end 136.656347 105.556347) (width 0.3) (layer "F.Cu") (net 4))
 (segment (start 135.35 94.55) (end 133.8 93) (width 0.3) (layer "F.Cu") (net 4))
 (segment (start 133.8 93) (end 129.42 93) (width 0.3) (layer "F.Cu") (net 4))
 (segment (start 136.687274 105.556347) (end 135.35 104.219073) (width 0.3) (layer "F.Cu") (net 4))
 (segment (start 135.7 111.070927) (end 135.7 116.36) (width 0.25) (layer "F.Cu") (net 16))
 (segment (start 135.7 116.36) (end 129 123.06) (width 0.25) (layer "F.Cu") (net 16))
 (segment (start 136.337044 110.433883) (end 135.7 111.070927) (width 0.25) (layer "F.Cu") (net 16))
 (segment (start 138.031798 119.391798) (end 146.78 128.14) (width 0.25) (layer "F.Cu") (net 19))
 (segment (start 138.031798 111.144581) (end 138.031798 119.391798) (width 0.25) (layer "F.Cu") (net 19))
 (segment (start 145.1 87.8) (end 146.48 87.8) (width 0.25) (layer "F.Cu") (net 35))
 (segment (start 139.95 103.991787) (end 139.95 92.95) (width 0.25) (layer "F.Cu") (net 35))
 (segment (start 139.95 92.95) (end 145.1 87.8) (width 0.25) (layer "F.Cu") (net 35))
 (segment (start 139.089313 104.852474) (end 139.95 103.991787) (width 0.25) (layer "F.Cu") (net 35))
 (segment (start 146.48 87.8) (end 146.78 87.5) (width 0.25) (layer "F.Cu") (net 35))
 (segment (start 145.604 98.836) (end 145.604 101.166927) (width 0.25) (layer "F.Cu") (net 31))
 (segment (start 146.78 97.66) (end 145.604 98.836) (width 0.25) (layer "F.Cu") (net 31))
 (segment (start 145.604 101.166927) (end 140.503883 106.267044) (width 0.25) (layer "F.Cu") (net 31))
 (segment (start 129 119.8) (end 129 120.52) (width 0.25) (layer "F.Cu") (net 15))
 (segment (start 135.983402 110.080241) (end 133 113.063643) (width 0.25) (layer "F.Cu") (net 15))
 (segment (start 133 116.52) (end 129 120.52) (width 0.25) (layer "F.Cu") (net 15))
 (segment (start 133 113.063643) (end 133 116.52) (width 0.25) (layer "F.Cu") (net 15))
 (segment (start 146.78 100.698213) (end 146.78 100.2) (width 0.25) (layer "F.Cu") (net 30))
 (segment (start 140.857526 106.620687) (end 146.78 100.698213) (width 0.25) (layer "F.Cu") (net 30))
 (segment (start 134.922474 109.019313) (end 131.041787 112.9) (width 0.25) (layer "F.Cu") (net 12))
 (segment (start 131.041787 112.9) (end 129 112.9) (width 0.25) (layer "F.Cu") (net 12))
 (segment (start 142.545671 106.974329) (end 146.78 102.74) (width 0.25) (layer "F.Cu") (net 29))
 (segment (start 141.211168 106.974329) (end 142.545671 106.974329) (width 0.25) (layer "F.Cu") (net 29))
 (segment (start 145.28 92.58) (end 146.78 92.58) (width 0.25) (layer "F.Cu") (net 33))
 (segment (start 145.25 92.55) (end 145.28 92.58) (width 0.25) (layer "F.Cu") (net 33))
 (segment (start 144.6 92.55) (end 145.25 92.55) (width 0.25) (layer "F.Cu") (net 33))
 (segment (start 139.796598 105.559759) (end 141.8 103.556357) (width 0.25) (layer "F.Cu") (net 33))
 (segment (start 141.8 95.35) (end 144.6 92.55) (width 0.25) (layer "F.Cu") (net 33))
 (segment (start 141.8 103.556357) (end 141.8 95.35) (width 0.25) (layer "F.Cu") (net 33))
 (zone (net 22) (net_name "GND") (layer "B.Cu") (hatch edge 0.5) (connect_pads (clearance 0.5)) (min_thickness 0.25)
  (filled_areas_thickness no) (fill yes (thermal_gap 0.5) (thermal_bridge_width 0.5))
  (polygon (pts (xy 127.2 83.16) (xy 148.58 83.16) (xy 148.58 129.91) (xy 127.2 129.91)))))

